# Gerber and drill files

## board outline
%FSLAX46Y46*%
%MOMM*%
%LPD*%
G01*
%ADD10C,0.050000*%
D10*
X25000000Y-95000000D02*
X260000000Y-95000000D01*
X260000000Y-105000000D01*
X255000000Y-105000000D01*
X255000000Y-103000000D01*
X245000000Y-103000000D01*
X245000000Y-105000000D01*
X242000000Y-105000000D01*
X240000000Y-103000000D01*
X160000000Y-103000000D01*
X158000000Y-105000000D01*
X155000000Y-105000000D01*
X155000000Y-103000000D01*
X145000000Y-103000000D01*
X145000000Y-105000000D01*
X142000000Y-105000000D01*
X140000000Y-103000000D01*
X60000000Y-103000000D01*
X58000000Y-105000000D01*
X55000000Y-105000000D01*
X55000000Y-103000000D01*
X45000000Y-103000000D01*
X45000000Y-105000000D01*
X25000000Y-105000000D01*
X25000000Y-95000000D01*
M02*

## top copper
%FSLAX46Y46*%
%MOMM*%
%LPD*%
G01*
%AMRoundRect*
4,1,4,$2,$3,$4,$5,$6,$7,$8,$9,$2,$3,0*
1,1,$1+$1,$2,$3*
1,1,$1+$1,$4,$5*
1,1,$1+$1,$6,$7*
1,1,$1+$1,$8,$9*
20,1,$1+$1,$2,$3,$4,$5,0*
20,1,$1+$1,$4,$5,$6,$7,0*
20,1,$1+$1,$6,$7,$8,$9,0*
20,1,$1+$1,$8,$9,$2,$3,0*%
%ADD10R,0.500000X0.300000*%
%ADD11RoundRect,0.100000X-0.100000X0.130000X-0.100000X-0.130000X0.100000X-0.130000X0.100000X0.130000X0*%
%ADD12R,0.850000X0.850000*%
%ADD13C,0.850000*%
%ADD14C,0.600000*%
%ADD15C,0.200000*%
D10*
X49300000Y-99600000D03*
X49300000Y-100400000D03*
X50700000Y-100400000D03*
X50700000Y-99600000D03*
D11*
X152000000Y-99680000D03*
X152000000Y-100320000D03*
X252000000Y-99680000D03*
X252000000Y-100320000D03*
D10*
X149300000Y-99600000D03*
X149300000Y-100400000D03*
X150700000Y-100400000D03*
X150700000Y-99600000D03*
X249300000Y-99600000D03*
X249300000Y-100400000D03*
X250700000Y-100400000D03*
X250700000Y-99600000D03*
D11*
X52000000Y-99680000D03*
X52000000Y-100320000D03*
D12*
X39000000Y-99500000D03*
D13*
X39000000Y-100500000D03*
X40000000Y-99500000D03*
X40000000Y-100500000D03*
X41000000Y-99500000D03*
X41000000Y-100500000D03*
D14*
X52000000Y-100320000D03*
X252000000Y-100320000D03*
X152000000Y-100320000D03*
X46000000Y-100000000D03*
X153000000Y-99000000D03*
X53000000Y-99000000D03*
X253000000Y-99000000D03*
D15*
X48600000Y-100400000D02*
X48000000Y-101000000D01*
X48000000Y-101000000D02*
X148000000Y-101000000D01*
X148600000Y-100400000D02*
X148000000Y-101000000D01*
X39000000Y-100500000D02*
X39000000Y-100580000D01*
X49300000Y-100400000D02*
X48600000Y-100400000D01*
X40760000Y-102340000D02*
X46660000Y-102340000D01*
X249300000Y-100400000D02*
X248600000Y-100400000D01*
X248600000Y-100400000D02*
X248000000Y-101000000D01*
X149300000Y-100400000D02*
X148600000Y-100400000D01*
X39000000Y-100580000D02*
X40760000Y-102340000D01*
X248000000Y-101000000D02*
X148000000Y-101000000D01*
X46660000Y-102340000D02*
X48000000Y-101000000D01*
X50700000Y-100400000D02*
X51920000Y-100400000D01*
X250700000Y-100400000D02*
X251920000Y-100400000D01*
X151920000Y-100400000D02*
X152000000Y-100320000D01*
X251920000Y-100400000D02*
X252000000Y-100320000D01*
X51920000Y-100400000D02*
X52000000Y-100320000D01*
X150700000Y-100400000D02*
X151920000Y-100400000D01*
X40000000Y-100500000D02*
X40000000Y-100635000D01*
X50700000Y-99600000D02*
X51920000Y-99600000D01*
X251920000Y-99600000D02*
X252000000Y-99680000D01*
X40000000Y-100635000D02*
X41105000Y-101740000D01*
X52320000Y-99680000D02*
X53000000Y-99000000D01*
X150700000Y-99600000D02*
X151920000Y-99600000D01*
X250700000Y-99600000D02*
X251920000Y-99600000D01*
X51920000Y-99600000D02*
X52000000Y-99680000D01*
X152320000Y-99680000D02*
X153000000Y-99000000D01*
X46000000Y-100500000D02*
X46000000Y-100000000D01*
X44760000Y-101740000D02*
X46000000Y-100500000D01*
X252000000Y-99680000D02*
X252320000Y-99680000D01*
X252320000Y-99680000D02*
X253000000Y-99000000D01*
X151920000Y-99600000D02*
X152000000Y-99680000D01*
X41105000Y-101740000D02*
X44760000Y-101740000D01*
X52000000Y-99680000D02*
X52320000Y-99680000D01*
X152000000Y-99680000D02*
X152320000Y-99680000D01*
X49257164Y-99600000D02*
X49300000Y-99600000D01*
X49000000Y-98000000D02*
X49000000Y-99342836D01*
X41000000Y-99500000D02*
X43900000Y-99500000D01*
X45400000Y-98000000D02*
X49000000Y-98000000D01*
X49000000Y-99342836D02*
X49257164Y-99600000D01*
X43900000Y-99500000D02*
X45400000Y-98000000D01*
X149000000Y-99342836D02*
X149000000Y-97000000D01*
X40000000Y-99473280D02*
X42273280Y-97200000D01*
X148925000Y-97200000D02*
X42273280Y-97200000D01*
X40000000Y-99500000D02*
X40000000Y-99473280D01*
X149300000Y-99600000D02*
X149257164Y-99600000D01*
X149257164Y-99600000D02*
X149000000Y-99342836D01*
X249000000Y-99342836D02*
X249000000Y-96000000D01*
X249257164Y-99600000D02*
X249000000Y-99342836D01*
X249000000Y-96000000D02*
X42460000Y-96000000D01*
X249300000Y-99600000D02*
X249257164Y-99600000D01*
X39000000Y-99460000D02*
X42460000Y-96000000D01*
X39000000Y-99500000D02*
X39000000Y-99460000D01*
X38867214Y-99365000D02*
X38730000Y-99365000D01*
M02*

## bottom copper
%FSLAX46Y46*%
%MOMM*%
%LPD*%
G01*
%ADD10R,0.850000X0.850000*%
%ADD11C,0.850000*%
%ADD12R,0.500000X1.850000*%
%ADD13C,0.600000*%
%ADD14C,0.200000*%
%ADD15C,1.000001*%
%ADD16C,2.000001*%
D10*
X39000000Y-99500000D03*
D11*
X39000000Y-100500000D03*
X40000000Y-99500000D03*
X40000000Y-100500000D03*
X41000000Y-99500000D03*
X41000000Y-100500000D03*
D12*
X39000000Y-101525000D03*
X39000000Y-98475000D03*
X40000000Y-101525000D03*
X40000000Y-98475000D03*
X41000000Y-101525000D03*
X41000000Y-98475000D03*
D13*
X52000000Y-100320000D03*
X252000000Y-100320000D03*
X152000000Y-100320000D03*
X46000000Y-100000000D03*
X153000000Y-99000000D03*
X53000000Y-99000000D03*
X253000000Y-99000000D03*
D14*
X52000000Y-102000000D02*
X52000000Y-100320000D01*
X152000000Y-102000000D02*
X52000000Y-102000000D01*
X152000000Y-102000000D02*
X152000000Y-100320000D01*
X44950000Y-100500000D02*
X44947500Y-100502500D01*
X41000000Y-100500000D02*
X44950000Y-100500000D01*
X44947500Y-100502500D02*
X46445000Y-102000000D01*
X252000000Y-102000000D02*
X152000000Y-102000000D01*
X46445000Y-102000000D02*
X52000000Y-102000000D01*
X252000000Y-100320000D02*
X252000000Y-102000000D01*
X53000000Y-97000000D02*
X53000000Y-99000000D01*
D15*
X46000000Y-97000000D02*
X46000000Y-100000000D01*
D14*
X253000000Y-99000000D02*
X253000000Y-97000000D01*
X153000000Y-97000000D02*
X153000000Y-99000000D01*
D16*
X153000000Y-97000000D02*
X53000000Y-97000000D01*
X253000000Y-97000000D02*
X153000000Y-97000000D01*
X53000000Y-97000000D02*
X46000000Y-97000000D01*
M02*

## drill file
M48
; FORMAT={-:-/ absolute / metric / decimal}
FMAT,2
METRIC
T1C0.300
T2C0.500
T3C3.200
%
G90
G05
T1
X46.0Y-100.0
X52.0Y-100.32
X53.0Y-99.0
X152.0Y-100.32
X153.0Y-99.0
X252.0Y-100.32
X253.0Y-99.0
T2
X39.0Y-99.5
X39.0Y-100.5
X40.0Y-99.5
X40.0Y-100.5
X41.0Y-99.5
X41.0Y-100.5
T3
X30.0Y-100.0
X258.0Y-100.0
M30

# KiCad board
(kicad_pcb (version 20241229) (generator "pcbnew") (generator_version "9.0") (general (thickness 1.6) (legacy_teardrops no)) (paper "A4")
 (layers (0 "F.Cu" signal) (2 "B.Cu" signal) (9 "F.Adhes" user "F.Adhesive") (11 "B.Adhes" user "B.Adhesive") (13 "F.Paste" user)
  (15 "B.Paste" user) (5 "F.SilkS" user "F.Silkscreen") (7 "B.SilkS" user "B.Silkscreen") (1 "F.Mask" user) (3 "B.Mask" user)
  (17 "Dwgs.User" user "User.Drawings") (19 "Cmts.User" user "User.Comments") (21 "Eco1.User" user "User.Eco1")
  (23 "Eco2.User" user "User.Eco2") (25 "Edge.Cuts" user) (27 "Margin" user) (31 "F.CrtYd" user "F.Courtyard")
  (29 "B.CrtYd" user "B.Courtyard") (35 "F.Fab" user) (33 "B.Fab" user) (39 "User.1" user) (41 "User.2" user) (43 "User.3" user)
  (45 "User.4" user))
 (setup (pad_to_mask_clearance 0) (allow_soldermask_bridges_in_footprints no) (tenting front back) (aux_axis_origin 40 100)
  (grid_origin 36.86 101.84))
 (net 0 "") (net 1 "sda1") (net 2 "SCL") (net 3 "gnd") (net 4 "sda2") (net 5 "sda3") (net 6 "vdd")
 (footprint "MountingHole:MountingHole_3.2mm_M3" (layer "F.Cu") (at 258 100)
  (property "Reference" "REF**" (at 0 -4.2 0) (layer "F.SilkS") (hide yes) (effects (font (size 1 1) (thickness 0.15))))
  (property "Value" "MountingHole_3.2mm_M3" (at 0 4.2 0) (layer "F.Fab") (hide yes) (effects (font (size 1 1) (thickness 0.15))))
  (pad "" np_thru_hole circle (at 0 0) (size 3.2 3.2) (drill 3.2) (layers "*.Cu" "*.Mask")))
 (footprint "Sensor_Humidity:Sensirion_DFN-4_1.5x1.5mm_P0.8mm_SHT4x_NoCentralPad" (layer "F.Cu") (at 50 100)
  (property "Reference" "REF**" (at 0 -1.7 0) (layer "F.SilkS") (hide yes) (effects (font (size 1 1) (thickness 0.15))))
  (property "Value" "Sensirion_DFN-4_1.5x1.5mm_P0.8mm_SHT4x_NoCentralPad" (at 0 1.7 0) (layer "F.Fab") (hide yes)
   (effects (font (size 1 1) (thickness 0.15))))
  (pad "1" smd rect (at -0.7 -0.4) (size 0.5 0.3) (layers "F.Cu" "F.Mask" "F.Paste") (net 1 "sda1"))
  (pad "2" smd rect (at -0.7 0.4) (size 0.5 0.3) (layers "F.Cu" "F.Mask" "F.Paste") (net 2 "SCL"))
  (pad "3" smd rect (at 0.7 0.4) (size 0.5 0.3) (layers "F.Cu" "F.Mask" "F.Paste"))
  (pad "4" smd rect (at 0.7 -0.4) (size 0.5 0.3) (layers "F.Cu" "F.Mask" "F.Paste") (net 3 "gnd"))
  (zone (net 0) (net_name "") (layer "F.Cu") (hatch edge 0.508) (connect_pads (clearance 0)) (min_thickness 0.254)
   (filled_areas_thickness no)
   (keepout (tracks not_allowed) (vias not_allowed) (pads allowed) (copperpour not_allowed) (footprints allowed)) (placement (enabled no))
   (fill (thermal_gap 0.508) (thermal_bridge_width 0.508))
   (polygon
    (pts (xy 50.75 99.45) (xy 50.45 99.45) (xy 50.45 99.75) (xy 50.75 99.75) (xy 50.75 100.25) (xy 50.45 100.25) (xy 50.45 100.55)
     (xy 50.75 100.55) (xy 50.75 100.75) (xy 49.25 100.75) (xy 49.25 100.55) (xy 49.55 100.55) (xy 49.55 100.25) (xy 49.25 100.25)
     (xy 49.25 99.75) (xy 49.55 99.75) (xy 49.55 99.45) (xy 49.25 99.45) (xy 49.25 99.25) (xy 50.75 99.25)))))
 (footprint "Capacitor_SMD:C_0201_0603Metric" (layer "F.Cu") (at 152 100 -90)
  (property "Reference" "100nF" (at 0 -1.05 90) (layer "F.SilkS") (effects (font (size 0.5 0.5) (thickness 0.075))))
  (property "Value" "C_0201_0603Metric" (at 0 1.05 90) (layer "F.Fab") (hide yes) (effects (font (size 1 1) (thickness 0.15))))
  (pad "" smd roundrect (at -0.345 0 270) (size 0.318 0.36) (layers "F.Paste") (roundrect_rratio 0.25))
  (pad "" smd roundrect (at 0.345 0 270) (size 0.318 0.36) (layers "F.Paste") (roundrect_rratio 0.25))
  (pad "1" smd roundrect (at -0.32 0 270) (size 0.46 0.4) (layers "F.Cu" "F.Mask") (roundrect_rratio 0.25))
  (pad "2" smd roundrect (at 0.32 0 270) (size 0.46 0.4) (layers "F.Cu" "F.Mask") (roundrect_rratio 0.25)))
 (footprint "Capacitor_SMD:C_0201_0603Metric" (layer "F.Cu") (at 252 100 -90)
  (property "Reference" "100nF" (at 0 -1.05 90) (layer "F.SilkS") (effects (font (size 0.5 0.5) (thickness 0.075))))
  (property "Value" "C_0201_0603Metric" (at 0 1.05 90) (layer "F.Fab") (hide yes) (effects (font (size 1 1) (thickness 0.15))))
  (pad "" smd roundrect (at -0.345 0 270) (size 0.318 0.36) (layers "F.Paste") (roundrect_rratio 0.25))
  (pad "" smd roundrect (at 0.345 0 270) (size 0.318 0.36) (layers "F.Paste") (roundrect_rratio 0.25))
  (pad "1" smd roundrect (at -0.32 0 270) (size 0.46 0.4) (layers "F.Cu" "F.Mask") (roundrect_rratio 0.25))
  (pad "2" smd roundrect (at 0.32 0 270) (size 0.46 0.4) (layers "F.Cu" "F.Mask") (roundrect_rratio 0.25)))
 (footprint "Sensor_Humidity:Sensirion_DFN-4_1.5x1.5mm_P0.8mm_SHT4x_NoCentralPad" (layer "F.Cu") (at 150 100)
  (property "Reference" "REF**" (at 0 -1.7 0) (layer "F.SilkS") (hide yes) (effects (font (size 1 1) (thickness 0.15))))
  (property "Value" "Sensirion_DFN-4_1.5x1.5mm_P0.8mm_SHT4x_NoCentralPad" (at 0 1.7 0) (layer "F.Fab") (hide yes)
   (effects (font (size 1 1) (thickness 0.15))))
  (pad "1" smd rect (at -0.7 -0.4) (size 0.5 0.3) (layers "F.Cu" "F.Mask" "F.Paste") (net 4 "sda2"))
  (pad "2" smd rect (at -0.7 0.4) (size 0.5 0.3) (layers "F.Cu" "F.Mask" "F.Paste") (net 2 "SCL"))
  (pad "3" smd rect (at 0.7 0.4) (size 0.5 0.3) (layers "F.Cu" "F.Mask" "F.Paste"))
  (pad "4" smd rect (at 0.7 -0.4) (size 0.5 0.3) (layers "F.Cu" "F.Mask" "F.Paste"))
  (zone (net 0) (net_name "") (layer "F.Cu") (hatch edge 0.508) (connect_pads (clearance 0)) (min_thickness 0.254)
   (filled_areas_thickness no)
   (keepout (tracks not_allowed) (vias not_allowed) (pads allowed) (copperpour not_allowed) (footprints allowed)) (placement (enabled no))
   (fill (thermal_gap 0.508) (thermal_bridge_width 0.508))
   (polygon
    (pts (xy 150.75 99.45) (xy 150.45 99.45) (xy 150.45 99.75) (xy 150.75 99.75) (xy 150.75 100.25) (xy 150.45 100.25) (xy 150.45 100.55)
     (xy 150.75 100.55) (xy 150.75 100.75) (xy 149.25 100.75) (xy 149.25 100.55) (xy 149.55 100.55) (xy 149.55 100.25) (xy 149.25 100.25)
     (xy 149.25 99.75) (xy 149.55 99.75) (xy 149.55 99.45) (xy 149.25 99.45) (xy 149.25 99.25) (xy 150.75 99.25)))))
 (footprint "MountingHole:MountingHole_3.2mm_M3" (layer "F.Cu") (at 30 100)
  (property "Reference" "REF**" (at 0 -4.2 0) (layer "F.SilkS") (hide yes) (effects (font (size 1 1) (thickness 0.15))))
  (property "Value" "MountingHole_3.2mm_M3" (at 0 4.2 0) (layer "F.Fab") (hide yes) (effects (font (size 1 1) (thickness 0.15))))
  (pad "" np_thru_hole circle (at 0 0) (size 3.2 3.2) (drill 3.2) (layers "*.Cu" "*.Mask")))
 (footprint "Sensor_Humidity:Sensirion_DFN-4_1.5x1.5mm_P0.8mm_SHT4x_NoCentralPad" (layer "F.Cu") (at 250 100)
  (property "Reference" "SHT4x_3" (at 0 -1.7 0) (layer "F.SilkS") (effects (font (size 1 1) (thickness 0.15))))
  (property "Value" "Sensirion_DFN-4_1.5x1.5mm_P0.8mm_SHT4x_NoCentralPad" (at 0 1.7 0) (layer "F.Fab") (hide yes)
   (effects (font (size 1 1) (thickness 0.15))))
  (pad "1" smd rect (at -0.7 -0.4) (size 0.5 0.3) (layers "F.Cu" "F.Mask" "F.Paste") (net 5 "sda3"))
  (pad "2" smd rect (at -0.7 0.4) (size 0.5 0.3) (layers "F.Cu" "F.Mask" "F.Paste") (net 2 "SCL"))
  (pad "3" smd rect (at 0.7 0.4) (size 0.5 0.3) (layers "F.Cu" "F.Mask" "F.Paste") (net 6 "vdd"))
  (pad "4" smd rect (at 0.7 -0.4) (size 0.5 0.3) (layers "F.Cu" "F.Mask" "F.Paste"))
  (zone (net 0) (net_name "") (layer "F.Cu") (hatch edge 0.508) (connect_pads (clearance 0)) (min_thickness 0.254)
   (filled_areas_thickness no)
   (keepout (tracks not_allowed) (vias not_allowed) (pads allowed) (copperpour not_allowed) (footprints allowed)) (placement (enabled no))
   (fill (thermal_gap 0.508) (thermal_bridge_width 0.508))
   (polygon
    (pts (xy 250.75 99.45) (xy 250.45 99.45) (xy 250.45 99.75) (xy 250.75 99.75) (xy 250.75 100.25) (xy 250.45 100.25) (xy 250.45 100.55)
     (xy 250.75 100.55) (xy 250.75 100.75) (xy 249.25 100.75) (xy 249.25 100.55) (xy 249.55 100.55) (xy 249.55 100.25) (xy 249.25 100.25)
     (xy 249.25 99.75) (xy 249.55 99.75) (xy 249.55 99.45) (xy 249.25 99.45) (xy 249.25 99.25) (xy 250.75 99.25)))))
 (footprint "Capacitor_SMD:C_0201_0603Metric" (layer "F.Cu") (at 52 100 -90)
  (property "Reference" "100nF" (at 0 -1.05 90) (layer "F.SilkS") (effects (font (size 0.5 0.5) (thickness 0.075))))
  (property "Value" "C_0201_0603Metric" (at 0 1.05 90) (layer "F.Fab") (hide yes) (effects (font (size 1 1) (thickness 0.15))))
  (pad "" smd roundrect (at -0.345 0 270) (size 0.318 0.36) (layers "F.Paste") (roundrect_rratio 0.25))
  (pad "" smd roundrect (at 0.345 0 270) (size 0.318 0.36) (layers "F.Paste") (roundrect_rratio 0.25))
  (pad "1" smd roundrect (at -0.32 0 270) (size 0.46 0.4) (layers "F.Cu" "F.Mask") (roundrect_rratio 0.25))
  (pad "2" smd roundrect (at 0.32 0 270) (size 0.46 0.4) (layers "F.Cu" "F.Mask") (roundrect_rratio 0.25)))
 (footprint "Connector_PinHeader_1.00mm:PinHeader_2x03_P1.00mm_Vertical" (layer "B.Cu") (at 39 99.5 -90)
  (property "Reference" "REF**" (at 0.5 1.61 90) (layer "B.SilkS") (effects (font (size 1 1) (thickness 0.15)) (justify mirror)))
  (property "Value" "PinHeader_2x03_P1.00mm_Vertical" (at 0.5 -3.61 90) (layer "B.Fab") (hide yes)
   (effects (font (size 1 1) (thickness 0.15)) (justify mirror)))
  (pad "1" thru_hole rect (at 0 0 270) (size 0.85 0.85) (drill 0.5) (layers "*.Cu" "*.Mask") (remove_unused_layers no) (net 5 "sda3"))
  (pad "2" thru_hole circle (at 1 0 270) (size 0.85 0.85) (drill 0.5) (layers "*.Cu" "*.Mask") (remove_unused_layers no) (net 2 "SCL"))
  (pad "3" thru_hole circle (at 0 -1 270) (size 0.85 0.85) (drill 0.5) (layers "*.Cu" "*.Mask") (remove_unused_layers no) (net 4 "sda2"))
  (pad "4" thru_hole circle (at 1 -1 270) (size 0.85 0.85) (drill 0.5) (layers "*.Cu" "*.Mask") (remove_unused_layers no) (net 3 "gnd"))
  (pad "5" thru_hole circle (at 0 -2 270) (size 0.85 0.85) (drill 0.5) (layers "*.Cu" "*.Mask") (remove_unused_layers no) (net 1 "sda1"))
  (pad "6" thru_hole circle (at 1 -2 270) (size 0.85 0.85) (drill 0.5) (layers "*.Cu" "*.Mask") (remove_unused_layers no) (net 6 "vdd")))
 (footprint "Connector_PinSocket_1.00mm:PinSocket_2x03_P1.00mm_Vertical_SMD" (layer "B.Cu") (at 40 100 -90)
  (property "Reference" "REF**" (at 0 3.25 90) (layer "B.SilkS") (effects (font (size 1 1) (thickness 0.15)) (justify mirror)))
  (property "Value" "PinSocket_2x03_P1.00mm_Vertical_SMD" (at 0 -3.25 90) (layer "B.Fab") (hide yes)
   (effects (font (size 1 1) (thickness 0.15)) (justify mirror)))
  (pad "1" smd rect (at 1.525 1 270) (size 1.85 0.5) (layers "B.Cu" "B.Mask" "B.Paste") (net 2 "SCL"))
  (pad "2" smd rect (at -1.525 1 270) (size 1.85 0.5) (layers "B.Cu" "B.Mask" "B.Paste") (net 5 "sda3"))
  (pad "3" smd rect (at 1.525 0 270) (size 1.85 0.5) (layers "B.Cu" "B.Mask" "B.Paste") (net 3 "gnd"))
  (pad "4" smd rect (at -1.525 0 270) (size 1.85 0.5) (layers "B.Cu" "B.Mask" "B.Paste") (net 4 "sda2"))
  (pad "5" smd rect (at 1.525 -1 270) (size 1.85 0.5) (layers "B.Cu" "B.Mask" "B.Paste") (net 6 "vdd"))
  (pad "6" smd rect (at -1.525 -1 270) (size 1.85 0.5) (layers "B.Cu" "B.Mask" "B.Paste") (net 1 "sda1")))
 (gr_poly
  (pts (xy 25 95) (xy 260 95) (xy 260 105) (xy 255 105) (xy 255 103) (xy 245 103) (xy 245 105) (xy 242 105) (xy 240 103) (xy 160 103)
   (xy 158 105) (xy 155 105) (xy 155 103) (xy 145 103) (xy 145 105) (xy 142 105) (xy 140 103) (xy 60 103) (xy 58 105) (xy 55 105)
   (xy 55 103) (xy 45 103) (xy 45 105) (xy 25 105))
  (stroke (width 0.05) (type solid)) (fill no) (layer "Edge.Cuts"))
 (segment (start 48.6 100.4) (end 48 101) (width 0.2) (layer "F.Cu") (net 2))
 (segment (start 48 101) (end 148 101) (width 0.2) (layer "F.Cu") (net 2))
 (segment (start 148.6 100.4) (end 148 101) (width 0.2) (layer "F.Cu") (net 2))
 (segment (start 39 100.5) (end 39 100.58) (width 0.2) (layer "F.Cu") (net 2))
 (segment (start 49.3 100.4) (end 48.6 100.4) (width 0.2) (layer "F.Cu") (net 2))
 (segment (start 40.76 102.34) (end 46.66 102.34) (width 0.2) (layer "F.Cu") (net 2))
 (segment (start 249.3 100.4) (end 248.6 100.4) (width 0.2) (layer "F.Cu") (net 2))
 (segment (start 248.6 100.4) (end 248 101) (width 0.2) (layer "F.Cu") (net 2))
 (segment (start 149.3 100.4) (end 148.6 100.4) (width 0.2) (layer "F.Cu") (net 2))
 (segment (start 39 100.58) (end 40.76 102.34) (width 0.2) (layer "F.Cu") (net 2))
 (segment (start 248 101) (end 148 101) (width 0.2) (layer "F.Cu") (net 2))
 (segment (start 46.66 102.34) (end 48 101) (width 0.2) (layer "F.Cu") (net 2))
 (segment (start 50.7 100.4) (end 51.92 100.4) (width 0.2) (layer "F.Cu") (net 6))
 (segment (start 250.7 100.4) (end 251.92 100.4) (width 0.2) (layer "F.Cu") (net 6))
 (segment (start 151.92 100.4) (end 152 100.32) (width 0.2) (layer "F.Cu") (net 6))
 (segment (start 251.92 100.4) (end 252 100.32) (width 0.2) (layer "F.Cu") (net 6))
 (segment (start 51.92 100.4) (end 52 100.32) (width 0.2) (layer "F.Cu") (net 6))
 (segment (start 150.7 100.4) (end 151.92 100.4) (width 0.2) (layer "F.Cu") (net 6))
 (via blind (at 52 100.32) (size 0.6) (drill 0.3) (layers "F.Cu" "B.Cu") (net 6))
 (via blind (at 252 100.32) (size 0.6) (drill 0.3) (layers "F.Cu" "B.Cu") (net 6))
 (via blind (at 152 100.32) (size 0.6) (drill 0.3) (layers "F.Cu" "B.Cu") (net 6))
 (segment (start 52 102) (end 52 100.32) (width 0.2) (layer "B.Cu") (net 6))
 (segment (start 152 102) (end 52 102) (width 0.2) (layer "B.Cu") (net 6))
 (segment (start 152 102) (end 152 100.32) (width 0.2) (layer "B.Cu") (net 6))
 (segment (start 44.95 100.5) (end 44.9475 100.5025) (width 0.2) (layer "B.Cu") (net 6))
 (segment (start 41 100.5) (end 44.95 100.5) (width 0.2) (layer "B.Cu") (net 6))
 (segment (start 44.9475 100.5025) (end 46.445 102) (width 0.2) (layer "B.Cu") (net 6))
 (segment (start 252 102) (end 152 102) (width 0.2) (layer "B.Cu") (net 6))
 (segment (start 46.445 102) (end 52 102) (width 0.2) (layer "B.Cu") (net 6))
 (segment (start 252 100.32) (end 252 102) (width 0.2) (layer "B.Cu") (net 6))
 (segment (start 40 100.5) (end 40 100.635) (width 0.2) (layer "F.Cu") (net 3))
 (segment (start 50.7 99.6) (end 51.92 99.6) (width 0.2) (layer "F.Cu") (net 3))
 (segment (start 251.92 99.6) (end 252 99.68) (width 0.2) (layer "F.Cu") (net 3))
 (segment (start 40 100.635) (end 41.105 101.74) (width 0.2) (layer "F.Cu") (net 3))
 (segment (start 52.32 99.68) (end 53 99) (width 0.2) (layer "F.Cu") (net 3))
 (segment (start 150.7 99.6) (end 151.92 99.6) (width 0.2) (layer "F.Cu") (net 3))
 (segment (start 250.7 99.6) (end 251.92 99.6) (width 0.2) (layer "F.Cu") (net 3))
 (segment (start 51.92 99.6) (end 52 99.68) (width 0.2) (layer "F.Cu") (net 3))
 (segment (start 152.32 99.68) (end 153 99) (width 0.2) (layer "F.Cu") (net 3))
 (segment (start 46 100.5) (end 46 100) (width 0.2) (layer "F.Cu") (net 3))
 (segment (start 44.76 101.74) (end 46 100.5) (width 0.2) (layer "F.Cu") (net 3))
 (segment (start 252 99.68) (end 252.32 99.68) (width 0.2) (layer "F.Cu") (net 3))
 (segment (start 252.32 99.68) (end 253 99) (width 0.2) (layer "F.Cu") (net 3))
 (segment (start 151.92 99.6) (end 152 99.68) (width 0.2) (layer "F.Cu") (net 3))
 (segment (start 41.105 101.74) (end 44.76 101.74) (width 0.2) (layer "F.Cu") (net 3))
 (segment (start 52 99.68) (end 52.32 99.68) (width 0.2) (layer "F.Cu") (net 3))
 (segment (start 152 99.68) (end 152.32 99.68) (width 0.2) (layer "F.Cu") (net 3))
 (via (at 46 100) (size 0.6) (drill 0.3) (layers "F.Cu" "B.Cu") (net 3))
 (via blind (at 153 99) (size 0.6) (drill 0.3) (layers "F.Cu" "B.Cu") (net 3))
 (via blind (at 53 99) (size 0.6) (drill 0.3) (layers "F.Cu" "B.Cu") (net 3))
 (via blind (at 253 99) (size 0.6) (drill 0.3) (layers "F.Cu" "B.Cu") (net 3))
 (segment (start 53 97) (end 53 99) (width 0.2) (layer "B.Cu") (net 3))
 (segment (start 46 97) (end 46 100) (width 1.000001) (layer "B.Cu") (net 3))
 (segment (start 253 99) (end 253 97) (width 0.2) (layer "B.Cu") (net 3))
 (segment (start 153 97) (end 153 99) (width 0.2) (layer "B.Cu") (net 3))
 (segment (start 153 97) (end 53 97) (width 2.000001) (layer "B.Cu") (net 3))
 (segment (start 253 97) (end 153 97) (width 2.000001) (layer "B.Cu") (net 3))
 (segment (start 53 97) (end 46 97) (width 2.000001) (layer "B.Cu") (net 3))
 (segment (start 49.257164 99.6) (end 49.3 99.6) (width 0.2) (layer "F.Cu") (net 1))
 (segment (start 49 98) (end 49 99.342836) (width 0.2) (layer "F.Cu") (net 1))
 (segment (start 41 99.5) (end 43.9 99.5) (width 0.2) (layer "F.Cu") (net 1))
 (segment (start 45.4 98) (end 49 98) (width 0.2) (layer "F.Cu") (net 1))
 (segment (start 49 99.342836) (end 49.257164 99.6) (width 0.2) (layer "F.Cu") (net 1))
 (segment (start 43.9 99.5) (end 45.4 98) (width 0.2) (layer "F.Cu") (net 1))
 (segment (start 149 99.342836) (end 149 97) (width 0.2) (layer "F.Cu") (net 4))
 (segment (start 40 99.47328) (end 42.27328 97.2) (width 0.2) (layer "F.Cu") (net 4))
 (segment (start 148.925 97.2) (end 42.27328 97.2) (width 0.2) (layer "F.Cu") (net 4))
 (segment (start 40 99.5) (end 40 99.47328) (width 0.2) (layer "F.Cu") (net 4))
 (segment (start 149.3 99.6) (end 149.257164 99.6) (width 0.2) (layer "F.Cu") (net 4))
 (segment (start 149.257164 99.6) (end 149 99.342836) (width 0.2) (layer "F.Cu") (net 4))
 (segment (start 249 99.342836) (end 249 96) (width 0.2) (layer "F.Cu") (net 5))
 (segment (start 249.257164 99.6) (end 249 99.342836) (width 0.2) (layer "F.Cu") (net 5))
 (segment (start 249 96) (end 42.46 96) (width 0.2) (layer "F.Cu") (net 5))
 (segment (start 249.3 99.6) (end 249.257164 99.6) (width 0.2) (layer "F.Cu") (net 5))
 (segment (start 39 99.46) (end 42.46 96) (width 0.2) (layer "F.Cu") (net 5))
 (segment (start 39 99.5) (end 39 99.46) (width 0.2) (layer "F.Cu") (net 5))
 (segment (start 38.867214 99.365) (end 38.73 99.365) (width 0.2) (layer "F.Cu") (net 5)))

